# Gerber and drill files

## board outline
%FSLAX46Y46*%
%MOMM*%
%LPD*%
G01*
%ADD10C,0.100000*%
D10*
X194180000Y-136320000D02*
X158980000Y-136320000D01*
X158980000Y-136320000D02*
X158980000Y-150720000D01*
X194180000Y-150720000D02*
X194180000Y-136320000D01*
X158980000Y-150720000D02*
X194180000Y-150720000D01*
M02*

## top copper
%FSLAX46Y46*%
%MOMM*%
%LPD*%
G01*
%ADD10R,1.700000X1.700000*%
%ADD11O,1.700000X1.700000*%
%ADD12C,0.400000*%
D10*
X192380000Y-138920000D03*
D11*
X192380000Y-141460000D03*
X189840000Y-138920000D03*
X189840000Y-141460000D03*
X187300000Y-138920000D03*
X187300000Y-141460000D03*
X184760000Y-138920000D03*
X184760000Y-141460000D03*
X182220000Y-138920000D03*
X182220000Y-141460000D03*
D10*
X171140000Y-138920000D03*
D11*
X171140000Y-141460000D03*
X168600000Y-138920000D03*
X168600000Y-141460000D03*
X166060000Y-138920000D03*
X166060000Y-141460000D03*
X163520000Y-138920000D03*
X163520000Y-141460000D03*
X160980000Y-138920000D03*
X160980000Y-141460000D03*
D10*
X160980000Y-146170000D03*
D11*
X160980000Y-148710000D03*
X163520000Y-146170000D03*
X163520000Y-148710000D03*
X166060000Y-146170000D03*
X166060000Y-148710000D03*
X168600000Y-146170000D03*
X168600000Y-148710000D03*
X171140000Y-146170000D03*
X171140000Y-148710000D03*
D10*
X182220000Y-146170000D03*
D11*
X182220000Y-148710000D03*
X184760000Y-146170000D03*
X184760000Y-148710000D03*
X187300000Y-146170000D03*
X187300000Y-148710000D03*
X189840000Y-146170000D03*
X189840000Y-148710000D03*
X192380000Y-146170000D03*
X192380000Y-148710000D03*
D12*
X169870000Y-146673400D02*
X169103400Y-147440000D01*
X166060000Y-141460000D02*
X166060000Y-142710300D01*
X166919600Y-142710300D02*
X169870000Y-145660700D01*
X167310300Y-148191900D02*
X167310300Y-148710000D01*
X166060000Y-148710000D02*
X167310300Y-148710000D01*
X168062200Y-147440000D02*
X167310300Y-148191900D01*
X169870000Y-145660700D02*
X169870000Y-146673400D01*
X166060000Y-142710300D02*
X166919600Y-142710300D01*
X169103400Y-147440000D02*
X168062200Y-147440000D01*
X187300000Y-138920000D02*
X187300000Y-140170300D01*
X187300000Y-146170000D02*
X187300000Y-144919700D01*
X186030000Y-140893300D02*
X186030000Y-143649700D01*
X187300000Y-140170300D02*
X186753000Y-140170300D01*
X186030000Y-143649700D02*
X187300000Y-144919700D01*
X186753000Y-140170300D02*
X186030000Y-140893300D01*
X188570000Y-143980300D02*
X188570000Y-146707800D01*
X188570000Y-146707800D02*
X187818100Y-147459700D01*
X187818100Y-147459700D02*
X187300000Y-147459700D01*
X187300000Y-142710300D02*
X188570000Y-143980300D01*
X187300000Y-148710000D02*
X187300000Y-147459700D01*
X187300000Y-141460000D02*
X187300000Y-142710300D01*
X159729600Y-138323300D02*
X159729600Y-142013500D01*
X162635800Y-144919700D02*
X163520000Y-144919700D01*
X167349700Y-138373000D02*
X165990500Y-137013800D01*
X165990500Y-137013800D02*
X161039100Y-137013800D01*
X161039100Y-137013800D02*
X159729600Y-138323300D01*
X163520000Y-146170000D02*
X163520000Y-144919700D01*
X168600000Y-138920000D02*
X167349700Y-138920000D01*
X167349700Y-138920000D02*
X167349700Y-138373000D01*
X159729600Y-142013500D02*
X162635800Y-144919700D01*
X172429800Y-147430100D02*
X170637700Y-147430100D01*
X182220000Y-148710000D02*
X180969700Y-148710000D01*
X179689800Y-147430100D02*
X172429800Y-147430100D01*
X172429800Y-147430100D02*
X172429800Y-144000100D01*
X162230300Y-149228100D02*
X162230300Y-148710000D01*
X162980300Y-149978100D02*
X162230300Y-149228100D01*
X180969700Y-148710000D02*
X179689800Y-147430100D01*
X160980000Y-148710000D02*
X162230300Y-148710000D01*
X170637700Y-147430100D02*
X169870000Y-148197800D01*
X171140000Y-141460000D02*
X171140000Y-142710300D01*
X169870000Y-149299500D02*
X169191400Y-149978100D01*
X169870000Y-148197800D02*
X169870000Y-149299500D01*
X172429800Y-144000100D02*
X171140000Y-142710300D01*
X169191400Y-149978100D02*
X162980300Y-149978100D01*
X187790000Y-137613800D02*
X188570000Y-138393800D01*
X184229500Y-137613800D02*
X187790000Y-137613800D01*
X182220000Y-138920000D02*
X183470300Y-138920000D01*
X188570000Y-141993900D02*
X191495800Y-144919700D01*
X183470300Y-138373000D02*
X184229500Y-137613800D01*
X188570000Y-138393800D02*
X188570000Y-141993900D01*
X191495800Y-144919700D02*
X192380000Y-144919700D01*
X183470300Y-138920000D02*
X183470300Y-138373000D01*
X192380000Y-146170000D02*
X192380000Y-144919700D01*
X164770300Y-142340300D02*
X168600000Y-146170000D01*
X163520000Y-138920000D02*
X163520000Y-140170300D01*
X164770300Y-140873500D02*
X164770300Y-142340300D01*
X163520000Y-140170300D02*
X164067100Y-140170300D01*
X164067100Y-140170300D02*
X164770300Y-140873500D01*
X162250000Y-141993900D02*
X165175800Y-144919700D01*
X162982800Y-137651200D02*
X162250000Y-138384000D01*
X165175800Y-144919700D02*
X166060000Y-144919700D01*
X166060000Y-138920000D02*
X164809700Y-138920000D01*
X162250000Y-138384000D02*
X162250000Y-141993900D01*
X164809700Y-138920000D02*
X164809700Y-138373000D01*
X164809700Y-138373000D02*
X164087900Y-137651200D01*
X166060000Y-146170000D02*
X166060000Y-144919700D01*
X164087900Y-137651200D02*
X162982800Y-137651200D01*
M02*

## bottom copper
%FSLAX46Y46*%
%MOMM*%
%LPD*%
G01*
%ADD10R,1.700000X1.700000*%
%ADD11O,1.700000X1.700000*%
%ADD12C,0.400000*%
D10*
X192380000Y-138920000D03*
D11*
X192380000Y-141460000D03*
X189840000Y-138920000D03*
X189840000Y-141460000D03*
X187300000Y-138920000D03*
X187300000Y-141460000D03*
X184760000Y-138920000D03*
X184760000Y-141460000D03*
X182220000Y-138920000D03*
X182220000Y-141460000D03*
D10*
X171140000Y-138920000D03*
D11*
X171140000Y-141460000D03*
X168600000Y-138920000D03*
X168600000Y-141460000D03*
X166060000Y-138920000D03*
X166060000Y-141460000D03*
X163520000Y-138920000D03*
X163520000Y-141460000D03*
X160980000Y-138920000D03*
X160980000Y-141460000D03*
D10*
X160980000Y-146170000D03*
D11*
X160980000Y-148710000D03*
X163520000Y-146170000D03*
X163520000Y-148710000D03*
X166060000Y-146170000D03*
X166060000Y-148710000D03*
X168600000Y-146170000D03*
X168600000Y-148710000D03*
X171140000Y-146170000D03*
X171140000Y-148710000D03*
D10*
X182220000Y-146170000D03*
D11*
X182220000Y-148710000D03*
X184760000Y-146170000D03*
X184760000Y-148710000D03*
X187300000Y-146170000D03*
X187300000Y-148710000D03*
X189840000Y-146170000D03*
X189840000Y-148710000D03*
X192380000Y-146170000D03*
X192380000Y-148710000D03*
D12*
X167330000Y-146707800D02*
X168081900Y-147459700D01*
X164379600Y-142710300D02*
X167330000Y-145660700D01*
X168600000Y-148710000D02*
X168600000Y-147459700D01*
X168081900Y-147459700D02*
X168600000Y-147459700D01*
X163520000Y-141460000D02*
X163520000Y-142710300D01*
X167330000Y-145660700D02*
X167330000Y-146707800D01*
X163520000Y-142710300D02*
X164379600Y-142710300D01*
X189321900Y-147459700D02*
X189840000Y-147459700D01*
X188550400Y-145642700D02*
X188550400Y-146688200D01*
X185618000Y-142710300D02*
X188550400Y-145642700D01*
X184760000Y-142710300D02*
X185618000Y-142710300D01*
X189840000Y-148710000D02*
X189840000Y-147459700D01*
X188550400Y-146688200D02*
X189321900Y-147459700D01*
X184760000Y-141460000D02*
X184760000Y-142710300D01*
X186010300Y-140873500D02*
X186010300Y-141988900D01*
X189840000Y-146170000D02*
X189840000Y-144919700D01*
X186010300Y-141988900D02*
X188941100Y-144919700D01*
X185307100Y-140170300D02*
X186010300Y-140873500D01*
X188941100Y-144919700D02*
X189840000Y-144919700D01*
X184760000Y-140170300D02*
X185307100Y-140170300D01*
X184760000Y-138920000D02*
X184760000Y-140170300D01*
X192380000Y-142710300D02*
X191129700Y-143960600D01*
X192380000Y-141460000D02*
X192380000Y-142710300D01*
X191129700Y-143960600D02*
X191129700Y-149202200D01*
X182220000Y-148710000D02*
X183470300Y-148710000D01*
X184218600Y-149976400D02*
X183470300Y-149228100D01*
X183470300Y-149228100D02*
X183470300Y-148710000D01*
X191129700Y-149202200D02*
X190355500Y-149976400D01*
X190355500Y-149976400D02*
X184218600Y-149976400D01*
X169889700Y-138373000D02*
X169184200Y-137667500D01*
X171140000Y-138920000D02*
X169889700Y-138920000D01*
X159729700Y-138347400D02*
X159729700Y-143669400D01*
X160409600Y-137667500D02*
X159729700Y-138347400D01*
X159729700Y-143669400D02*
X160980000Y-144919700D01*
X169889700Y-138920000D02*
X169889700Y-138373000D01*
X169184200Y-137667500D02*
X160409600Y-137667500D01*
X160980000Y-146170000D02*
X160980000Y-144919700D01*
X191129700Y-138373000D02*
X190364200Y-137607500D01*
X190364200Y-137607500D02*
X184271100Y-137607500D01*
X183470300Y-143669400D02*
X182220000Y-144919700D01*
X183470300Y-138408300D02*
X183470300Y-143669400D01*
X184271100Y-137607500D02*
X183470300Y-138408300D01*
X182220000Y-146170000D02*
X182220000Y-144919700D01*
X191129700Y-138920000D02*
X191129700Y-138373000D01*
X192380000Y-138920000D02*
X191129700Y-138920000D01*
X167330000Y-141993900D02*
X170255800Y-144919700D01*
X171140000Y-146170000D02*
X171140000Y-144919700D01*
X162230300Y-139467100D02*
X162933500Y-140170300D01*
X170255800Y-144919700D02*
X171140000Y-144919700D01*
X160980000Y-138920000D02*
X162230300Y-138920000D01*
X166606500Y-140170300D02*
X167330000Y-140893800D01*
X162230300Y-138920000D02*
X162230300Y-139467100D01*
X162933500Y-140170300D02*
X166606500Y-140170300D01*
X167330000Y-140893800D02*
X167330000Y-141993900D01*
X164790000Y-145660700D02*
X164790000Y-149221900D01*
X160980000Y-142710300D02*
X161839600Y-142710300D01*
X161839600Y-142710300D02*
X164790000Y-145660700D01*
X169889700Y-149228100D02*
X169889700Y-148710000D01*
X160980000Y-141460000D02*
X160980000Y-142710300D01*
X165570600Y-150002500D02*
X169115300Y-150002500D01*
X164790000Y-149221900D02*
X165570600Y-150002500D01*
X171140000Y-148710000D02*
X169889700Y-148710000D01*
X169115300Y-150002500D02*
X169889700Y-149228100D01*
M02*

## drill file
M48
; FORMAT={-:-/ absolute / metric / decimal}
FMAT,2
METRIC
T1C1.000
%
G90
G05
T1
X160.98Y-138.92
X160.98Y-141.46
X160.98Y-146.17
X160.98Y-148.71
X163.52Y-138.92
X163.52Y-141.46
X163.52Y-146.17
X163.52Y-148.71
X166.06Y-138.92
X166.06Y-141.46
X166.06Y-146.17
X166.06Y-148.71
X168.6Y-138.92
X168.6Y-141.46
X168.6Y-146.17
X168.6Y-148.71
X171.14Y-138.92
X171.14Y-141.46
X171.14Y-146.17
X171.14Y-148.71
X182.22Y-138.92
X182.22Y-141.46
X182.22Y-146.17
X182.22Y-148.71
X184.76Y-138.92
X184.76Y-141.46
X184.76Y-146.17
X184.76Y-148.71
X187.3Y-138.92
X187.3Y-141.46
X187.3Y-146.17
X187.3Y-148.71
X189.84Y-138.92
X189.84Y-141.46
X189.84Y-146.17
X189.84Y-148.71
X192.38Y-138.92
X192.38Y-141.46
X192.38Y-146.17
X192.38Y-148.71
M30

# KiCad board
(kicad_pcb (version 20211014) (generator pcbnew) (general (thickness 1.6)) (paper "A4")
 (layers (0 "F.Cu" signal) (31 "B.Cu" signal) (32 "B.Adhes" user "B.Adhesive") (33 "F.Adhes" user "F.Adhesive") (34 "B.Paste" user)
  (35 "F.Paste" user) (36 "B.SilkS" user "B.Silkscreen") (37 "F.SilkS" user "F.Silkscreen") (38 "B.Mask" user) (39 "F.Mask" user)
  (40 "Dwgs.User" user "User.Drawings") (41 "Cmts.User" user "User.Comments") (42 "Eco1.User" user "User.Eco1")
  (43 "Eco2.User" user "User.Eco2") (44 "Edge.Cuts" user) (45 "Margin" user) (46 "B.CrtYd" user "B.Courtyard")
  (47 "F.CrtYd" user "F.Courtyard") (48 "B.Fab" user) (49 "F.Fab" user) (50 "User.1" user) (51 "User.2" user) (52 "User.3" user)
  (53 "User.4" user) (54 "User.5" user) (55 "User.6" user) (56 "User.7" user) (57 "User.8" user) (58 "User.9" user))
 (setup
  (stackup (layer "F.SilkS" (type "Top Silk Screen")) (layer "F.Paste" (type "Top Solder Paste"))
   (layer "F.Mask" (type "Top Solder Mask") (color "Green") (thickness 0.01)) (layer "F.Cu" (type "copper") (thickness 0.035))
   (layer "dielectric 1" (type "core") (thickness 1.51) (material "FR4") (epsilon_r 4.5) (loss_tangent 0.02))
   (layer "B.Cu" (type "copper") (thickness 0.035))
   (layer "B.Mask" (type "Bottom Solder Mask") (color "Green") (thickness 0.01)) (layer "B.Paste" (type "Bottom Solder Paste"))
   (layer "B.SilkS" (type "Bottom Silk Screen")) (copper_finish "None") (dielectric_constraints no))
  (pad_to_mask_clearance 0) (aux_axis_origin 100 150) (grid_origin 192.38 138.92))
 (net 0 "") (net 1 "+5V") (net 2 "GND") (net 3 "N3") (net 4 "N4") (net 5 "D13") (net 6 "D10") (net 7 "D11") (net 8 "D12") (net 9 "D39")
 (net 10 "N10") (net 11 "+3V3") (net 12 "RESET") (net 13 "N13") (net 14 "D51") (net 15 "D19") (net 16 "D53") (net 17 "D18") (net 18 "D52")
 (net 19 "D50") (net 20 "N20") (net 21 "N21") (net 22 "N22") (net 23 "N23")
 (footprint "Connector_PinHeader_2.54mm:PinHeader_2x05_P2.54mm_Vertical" (layer "F.Cu") (at 192.38 138.92 -90)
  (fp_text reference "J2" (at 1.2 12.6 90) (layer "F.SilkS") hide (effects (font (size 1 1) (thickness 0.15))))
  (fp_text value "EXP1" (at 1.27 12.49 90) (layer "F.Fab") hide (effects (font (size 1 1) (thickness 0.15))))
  (pad "1" thru_hole rect locked (at 0 0 270) (size 1.7 1.7) (drill 1) (layers *.Cu *.Mask) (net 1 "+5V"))
  (pad "2" thru_hole oval locked (at 2.54 0 270) (size 1.7 1.7) (drill 1) (layers *.Cu *.Mask) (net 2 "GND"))
  (pad "3" thru_hole oval locked (at 0 2.54 270) (size 1.7 1.7) (drill 1) (layers *.Cu *.Mask) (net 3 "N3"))
  (pad "4" thru_hole oval locked (at 2.54 2.54 270) (size 1.7 1.7) (drill 1) (layers *.Cu *.Mask) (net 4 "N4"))
  (pad "5" thru_hole oval locked (at 0 5.08 270) (size 1.7 1.7) (drill 1) (layers *.Cu *.Mask) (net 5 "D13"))
  (pad "6" thru_hole oval locked (at 2.54 5.08 270) (size 1.7 1.7) (drill 1) (layers *.Cu *.Mask) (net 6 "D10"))
  (pad "7" thru_hole oval locked (at 0 7.62 270) (size 1.7 1.7) (drill 1) (layers *.Cu *.Mask) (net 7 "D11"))
  (pad "8" thru_hole oval locked (at 2.54 7.62 270) (size 1.7 1.7) (drill 1) (layers *.Cu *.Mask) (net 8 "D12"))
  (pad "9" thru_hole oval locked (at 0 10.16 270) (size 1.7 1.7) (drill 1) (layers *.Cu *.Mask) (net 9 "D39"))
  (pad "10" thru_hole oval locked (at 2.54 10.16 270) (size 1.7 1.7) (drill 1) (layers *.Cu *.Mask) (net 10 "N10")))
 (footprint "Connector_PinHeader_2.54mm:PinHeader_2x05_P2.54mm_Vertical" (layer "F.Cu") (at 171.14 138.92 -90)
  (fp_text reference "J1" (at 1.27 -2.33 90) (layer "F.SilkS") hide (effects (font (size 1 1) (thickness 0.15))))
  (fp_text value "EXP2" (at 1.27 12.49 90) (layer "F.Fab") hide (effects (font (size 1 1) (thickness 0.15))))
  (pad "1" thru_hole rect locked (at 0 0 270) (size 1.7 1.7) (drill 1) (layers *.Cu *.Mask) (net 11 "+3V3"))
  (pad "2" thru_hole oval locked (at 2.54 0 270) (size 1.7 1.7) (drill 1) (layers *.Cu *.Mask) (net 2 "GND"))
  (pad "3" thru_hole oval locked (at 0 2.54 270) (size 1.7 1.7) (drill 1) (layers *.Cu *.Mask) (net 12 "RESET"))
  (pad "4" thru_hole oval locked (at 2.54 2.54 270) (size 1.7 1.7) (drill 1) (layers *.Cu *.Mask) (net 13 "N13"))
  (pad "5" thru_hole oval locked (at 0 5.08 270) (size 1.7 1.7) (drill 1) (layers *.Cu *.Mask) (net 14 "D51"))
  (pad "6" thru_hole oval locked (at 2.54 5.08 270) (size 1.7 1.7) (drill 1) (layers *.Cu *.Mask) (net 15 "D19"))
  (pad "7" thru_hole oval locked (at 0 7.62 270) (size 1.7 1.7) (drill 1) (layers *.Cu *.Mask) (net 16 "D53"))
  (pad "8" thru_hole oval locked (at 2.54 7.62 270) (size 1.7 1.7) (drill 1) (layers *.Cu *.Mask) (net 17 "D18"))
  (pad "9" thru_hole oval locked (at 0 10.16 270) (size 1.7 1.7) (drill 1) (layers *.Cu *.Mask) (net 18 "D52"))
  (pad "10" thru_hole oval locked (at 2.54 10.16 270) (size 1.7 1.7) (drill 1) (layers *.Cu *.Mask) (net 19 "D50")))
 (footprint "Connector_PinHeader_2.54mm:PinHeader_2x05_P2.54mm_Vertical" (layer "B.Cu") (at 160.98 146.17 -90)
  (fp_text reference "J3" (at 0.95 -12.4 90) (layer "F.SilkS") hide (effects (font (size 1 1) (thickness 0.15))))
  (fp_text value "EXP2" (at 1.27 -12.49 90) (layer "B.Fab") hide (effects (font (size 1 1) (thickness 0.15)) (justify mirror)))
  (pad "1" thru_hole rect locked (at 0 0 270) (size 1.7 1.7) (drill 1) (layers *.Cu *.Mask) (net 11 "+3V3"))
  (pad "2" thru_hole oval locked (at 2.54 0 270) (size 1.7 1.7) (drill 1) (layers *.Cu *.Mask) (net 2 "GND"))
  (pad "3" thru_hole oval locked (at 0 -2.54 270) (size 1.7 1.7) (drill 1) (layers *.Cu *.Mask) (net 12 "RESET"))
  (pad "4" thru_hole oval locked (at 2.54 -2.54 270) (size 1.7 1.7) (drill 1) (layers *.Cu *.Mask) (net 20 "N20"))
  (pad "5" thru_hole oval locked (at 0 -5.08 270) (size 1.7 1.7) (drill 1) (layers *.Cu *.Mask) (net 14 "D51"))
  (pad "6" thru_hole oval locked (at 2.54 -5.08 270) (size 1.7 1.7) (drill 1) (layers *.Cu *.Mask) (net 15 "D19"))
  (pad "7" thru_hole oval locked (at 0 -7.62 270) (size 1.7 1.7) (drill 1) (layers *.Cu *.Mask) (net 16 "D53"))
  (pad "8" thru_hole oval locked (at 2.54 -7.62 270) (size 1.7 1.7) (drill 1) (layers *.Cu *.Mask) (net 17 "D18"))
  (pad "9" thru_hole oval locked (at 0 -10.16 270) (size 1.7 1.7) (drill 1) (layers *.Cu *.Mask) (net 18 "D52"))
  (pad "10" thru_hole oval locked (at 2.54 -10.16 270) (size 1.7 1.7) (drill 1) (layers *.Cu *.Mask) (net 19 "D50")))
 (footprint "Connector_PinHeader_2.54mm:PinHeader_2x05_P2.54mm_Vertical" (layer "B.Cu") (at 182.22 146.17 -90)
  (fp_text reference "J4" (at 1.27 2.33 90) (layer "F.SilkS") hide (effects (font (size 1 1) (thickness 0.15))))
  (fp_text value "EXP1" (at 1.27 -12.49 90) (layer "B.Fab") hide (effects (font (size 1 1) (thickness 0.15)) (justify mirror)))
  (pad "1" thru_hole rect locked (at 0 0 270) (size 1.7 1.7) (drill 1) (layers *.Cu *.Mask) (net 1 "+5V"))
  (pad "2" thru_hole oval locked (at 2.54 0 270) (size 1.7 1.7) (drill 1) (layers *.Cu *.Mask) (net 2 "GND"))
  (pad "3" thru_hole oval locked (at 0 -2.54 270) (size 1.7 1.7) (drill 1) (layers *.Cu *.Mask) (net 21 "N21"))
  (pad "4" thru_hole oval locked (at 2.54 -2.54 270) (size 1.7 1.7) (drill 1) (layers *.Cu *.Mask) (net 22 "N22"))
  (pad "5" thru_hole oval locked (at 0 -5.08 270) (size 1.7 1.7) (drill 1) (layers *.Cu *.Mask) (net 5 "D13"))
  (pad "6" thru_hole oval locked (at 2.54 -5.08 270) (size 1.7 1.7) (drill 1) (layers *.Cu *.Mask) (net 6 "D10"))
  (pad "7" thru_hole oval locked (at 0 -7.62 270) (size 1.7 1.7) (drill 1) (layers *.Cu *.Mask) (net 7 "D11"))
  (pad "8" thru_hole oval locked (at 2.54 -7.62 270) (size 1.7 1.7) (drill 1) (layers *.Cu *.Mask) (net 8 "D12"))
  (pad "9" thru_hole oval locked (at 0 -10.16 270) (size 1.7 1.7) (drill 1) (layers *.Cu *.Mask) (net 9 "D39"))
  (pad "10" thru_hole oval locked (at 2.54 -10.16 270) (size 1.7 1.7) (drill 1) (layers *.Cu *.Mask) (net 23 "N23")))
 (gr_line (start 194.18 136.32) (end 158.98 136.32) (layer "Edge.Cuts") (width 0.1))
 (gr_line (start 158.98 136.32) (end 158.98 150.72) (layer "Edge.Cuts") (width 0.1))
 (gr_line (start 194.18 150.72) (end 194.18 136.32) (layer "Edge.Cuts") (width 0.1))
 (gr_line (start 158.98 150.72) (end 194.18 150.72) (layer "Edge.Cuts") (width 0.1))
 (segment (start 167.33 146.7078) (end 168.0819 147.4597) (width 0.4) (layer "B.Cu") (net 17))
 (segment (start 164.3796 142.7103) (end 167.33 145.6607) (width 0.4) (layer "B.Cu") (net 17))
 (segment (start 168.6 148.71) (end 168.6 147.4597) (width 0.4) (layer "B.Cu") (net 17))
 (segment (start 168.0819 147.4597) (end 168.6 147.4597) (width 0.4) (layer "B.Cu") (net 17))
 (segment (start 163.52 141.46) (end 163.52 142.7103) (width 0.4) (layer "B.Cu") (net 17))
 (segment (start 167.33 145.6607) (end 167.33 146.7078) (width 0.4) (layer "B.Cu") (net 17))
 (segment (start 163.52 142.7103) (end 164.3796 142.7103) (width 0.4) (layer "B.Cu") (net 17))
 (segment (start 169.87 146.6734) (end 169.1034 147.44) (width 0.4) (layer "F.Cu") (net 15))
 (segment (start 166.06 141.46) (end 166.06 142.7103) (width 0.4) (layer "F.Cu") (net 15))
 (segment (start 166.9196 142.7103) (end 169.87 145.6607) (width 0.4) (layer "F.Cu") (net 15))
 (segment (start 167.3103 148.1919) (end 167.3103 148.71) (width 0.4) (layer "F.Cu") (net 15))
 (segment (start 166.06 148.71) (end 167.3103 148.71) (width 0.4) (layer "F.Cu") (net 15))
 (segment (start 168.0622 147.44) (end 167.3103 148.1919) (width 0.4) (layer "F.Cu") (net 15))
 (segment (start 169.87 145.6607) (end 169.87 146.6734) (width 0.4) (layer "F.Cu") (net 15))
 (segment (start 166.06 142.7103) (end 166.9196 142.7103) (width 0.4) (layer "F.Cu") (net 15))
 (segment (start 169.1034 147.44) (end 168.0622 147.44) (width 0.4) (layer "F.Cu") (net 15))
 (segment (start 189.3219 147.4597) (end 189.84 147.4597) (width 0.4) (layer "B.Cu") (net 8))
 (segment (start 188.5504 145.6427) (end 188.5504 146.6882) (width 0.4) (layer "B.Cu") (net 8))
 (segment (start 185.618 142.7103) (end 188.5504 145.6427) (width 0.4) (layer "B.Cu") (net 8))
 (segment (start 184.76 142.7103) (end 185.618 142.7103) (width 0.4) (layer "B.Cu") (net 8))
 (segment (start 189.84 148.71) (end 189.84 147.4597) (width 0.4) (layer "B.Cu") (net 8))
 (segment (start 188.5504 146.6882) (end 189.3219 147.4597) (width 0.4) (layer "B.Cu") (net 8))
 (segment (start 184.76 141.46) (end 184.76 142.7103) (width 0.4) (layer "B.Cu") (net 8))
 (segment (start 187.3 138.92) (end 187.3 140.1703) (width 0.4) (layer "F.Cu") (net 5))
 (segment (start 187.3 146.17) (end 187.3 144.9197) (width 0.4) (layer "F.Cu") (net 5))
 (segment (start 186.03 140.8933) (end 186.03 143.6497) (width 0.4) (layer "F.Cu") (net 5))
 (segment (start 187.3 140.1703) (end 186.753 140.1703) (width 0.4) (layer "F.Cu") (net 5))
 (segment (start 186.03 143.6497) (end 187.3 144.9197) (width 0.4) (layer "F.Cu") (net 5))
 (segment (start 186.753 140.1703) (end 186.03 140.8933) (width 0.4) (layer "F.Cu") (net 5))
 (segment (start 188.57 143.9803) (end 188.57 146.7078) (width 0.4) (layer "F.Cu") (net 6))
 (segment (start 188.57 146.7078) (end 187.8181 147.4597) (width 0.4) (layer "F.Cu") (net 6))
 (segment (start 187.8181 147.4597) (end 187.3 147.4597) (width 0.4) (layer "F.Cu") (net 6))
 (segment (start 187.3 142.7103) (end 188.57 143.9803) (width 0.4) (layer "F.Cu") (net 6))
 (segment (start 187.3 148.71) (end 187.3 147.4597) (width 0.4) (layer "F.Cu") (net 6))
 (segment (start 187.3 141.46) (end 187.3 142.7103) (width 0.4) (layer "F.Cu") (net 6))
 (segment (start 186.0103 140.8735) (end 186.0103 141.9889) (width 0.4) (layer "B.Cu") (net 7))
 (segment (start 189.84 146.17) (end 189.84 144.9197) (width 0.4) (layer "B.Cu") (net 7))
 (segment (start 186.0103 141.9889) (end 188.9411 144.9197) (width 0.4) (layer "B.Cu") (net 7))
 (segment (start 185.3071 140.1703) (end 186.0103 140.8735) (width 0.4) (layer "B.Cu") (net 7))
 (segment (start 188.9411 144.9197) (end 189.84 144.9197) (width 0.4) (layer "B.Cu") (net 7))
 (segment (start 184.76 140.1703) (end 185.3071 140.1703) (width 0.4) (layer "B.Cu") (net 7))
 (segment (start 184.76 138.92) (end 184.76 140.1703) (width 0.4) (layer "B.Cu") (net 7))
 (segment (start 159.7296 138.3233) (end 159.7296 142.0135) (width 0.4) (layer "F.Cu") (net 12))
 (segment (start 162.6358 144.9197) (end 163.52 144.9197) (width 0.4) (layer "F.Cu") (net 12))
 (segment (start 167.3497 138.373) (end 165.9905 137.0138) (width 0.4) (layer "F.Cu") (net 12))
 (segment (start 165.9905 137.0138) (end 161.0391 137.0138) (width 0.4) (layer "F.Cu") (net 12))
 (segment (start 161.0391 137.0138) (end 159.7296 138.3233) (width 0.4) (layer "F.Cu") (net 12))
 (segment (start 163.52 146.17) (end 163.52 144.9197) (width 0.4) (layer "F.Cu") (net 12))
 (segment (start 168.6 138.92) (end 167.3497 138.92) (width 0.4) (layer "F.Cu") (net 12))
 (segment (start 167.3497 138.92) (end 167.3497 138.373) (width 0.4) (layer "F.Cu") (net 12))
 (segment (start 159.7296 142.0135) (end 162.6358 144.9197) (width 0.4) (layer "F.Cu") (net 12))
 (segment (start 172.4298 147.4301) (end 170.6377 147.4301) (width 0.4) (layer "F.Cu") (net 2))
 (segment (start 182.22 148.71) (end 180.9697 148.71) (width 0.4) (layer "F.Cu") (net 2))
 (segment (start 179.6898 147.4301) (end 172.4298 147.4301) (width 0.4) (layer "F.Cu") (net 2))
 (segment (start 172.4298 147.4301) (end 172.4298 144.0001) (width 0.4) (layer "F.Cu") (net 2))
 (segment (start 162.2303 149.2281) (end 162.2303 148.71) (width 0.4) (layer "F.Cu") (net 2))
 (segment (start 162.9803 149.9781) (end 162.2303 149.2281) (width 0.4) (layer "F.Cu") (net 2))
 (segment (start 180.9697 148.71) (end 179.6898 147.4301) (width 0.4) (layer "F.Cu") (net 2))
 (segment (start 160.98 148.71) (end 162.2303 148.71) (width 0.4) (layer "F.Cu") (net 2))
 (segment (start 170.6377 147.4301) (end 169.87 148.1978) (width 0.4) (layer "F.Cu") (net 2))
 (segment (start 171.14 141.46) (end 171.14 142.7103) (width 0.4) (layer "F.Cu") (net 2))
 (segment (start 169.87 149.2995) (end 169.1914 149.9781) (width 0.4) (layer "F.Cu") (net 2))
 (segment (start 169.87 148.1978) (end 169.87 149.2995) (width 0.4) (layer "F.Cu") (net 2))
 (segment (start 172.4298 144.0001) (end 171.14 142.7103) (width 0.4) (layer "F.Cu") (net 2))
 (segment (start 169.1914 149.9781) (end 162.9803 149.9781) (width 0.4) (layer "F.Cu") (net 2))
 (segment (start 192.38 142.7103) (end 191.1297 143.9606) (width 0.4) (layer "B.Cu") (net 2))
 (segment (start 192.38 141.46) (end 192.38 142.7103) (width 0.4) (layer "B.Cu") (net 2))
 (segment (start 191.1297 143.9606) (end 191.1297 149.2022) (width 0.4) (layer "B.Cu") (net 2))
 (segment (start 182.22 148.71) (end 183.4703 148.71) (width 0.4) (layer "B.Cu") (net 2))
 (segment (start 184.2186 149.9764) (end 183.4703 149.2281) (width 0.4) (layer "B.Cu") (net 2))
 (segment (start 183.4703 149.2281) (end 183.4703 148.71) (width 0.4) (layer "B.Cu") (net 2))
 (segment (start 191.1297 149.2022) (end 190.3555 149.9764) (width 0.4) (layer "B.Cu") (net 2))
 (segment (start 190.3555 149.9764) (end 184.2186 149.9764) (width 0.4) (layer "B.Cu") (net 2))
 (segment (start 187.79 137.6138) (end 188.57 138.3938) (width 0.4) (layer "F.Cu") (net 9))
 (segment (start 184.2295 137.6138) (end 187.79 137.6138) (width 0.4) (layer "F.Cu") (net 9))
 (segment (start 182.22 138.92) (end 183.4703 138.92) (width 0.4) (layer "F.Cu") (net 9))
 (segment (start 188.57 141.9939) (end 191.4958 144.9197) (width 0.4) (layer "F.Cu") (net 9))
 (segment (start 183.4703 138.373) (end 184.2295 137.6138) (width 0.4) (layer "F.Cu") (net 9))
 (segment (start 188.57 138.3938) (end 188.57 141.9939) (width 0.4) (layer "F.Cu") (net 9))
 (segment (start 191.4958 144.9197) (end 192.38 144.9197) (width 0.4) (layer "F.Cu") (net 9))
 (segment (start 183.4703 138.92) (end 183.4703 138.373) (width 0.4) (layer "F.Cu") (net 9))
 (segment (start 192.38 146.17) (end 192.38 144.9197) (width 0.4) (layer "F.Cu") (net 9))
 (segment (start 169.8897 138.373) (end 169.1842 137.6675) (width 0.4) (layer "B.Cu") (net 11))
 (segment (start 171.14 138.92) (end 169.8897 138.92) (width 0.4) (layer "B.Cu") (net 11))
 (segment (start 159.7297 138.3474) (end 159.7297 143.6694) (width 0.4) (layer "B.Cu") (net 11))
 (segment (start 160.4096 137.6675) (end 159.7297 138.3474) (width 0.4) (layer "B.Cu") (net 11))
 (segment (start 159.7297 143.6694) (end 160.98 144.9197) (width 0.4) (layer "B.Cu") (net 11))
 (segment (start 169.8897 138.92) (end 169.8897 138.373) (width 0.4) (layer "B.Cu") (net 11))
 (segment (start 169.1842 137.6675) (end 160.4096 137.6675) (width 0.4) (layer "B.Cu") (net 11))
 (segment (start 160.98 146.17) (end 160.98 144.9197) (width 0.4) (layer "B.Cu") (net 11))
 (segment (start 191.1297 138.373) (end 190.3642 137.6075) (width 0.4) (layer "B.Cu") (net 1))
 (segment (start 190.3642 137.6075) (end 184.2711 137.6075) (width 0.4) (layer "B.Cu") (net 1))
 (segment (start 183.4703 143.6694) (end 182.22 144.9197) (width 0.4) (layer "B.Cu") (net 1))
 (segment (start 183.4703 138.4083) (end 183.4703 143.6694) (width 0.4) (layer "B.Cu") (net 1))
 (segment (start 184.2711 137.6075) (end 183.4703 138.4083) (width 0.4) (layer "B.Cu") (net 1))
 (segment (start 182.22 146.17) (end 182.22 144.9197) (width 0.4) (layer "B.Cu") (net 1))
 (segment (start 191.1297 138.92) (end 191.1297 138.373) (width 0.4) (layer "B.Cu") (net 1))
 (segment (start 192.38 138.92) (end 191.1297 138.92) (width 0.4) (layer "B.Cu") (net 1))
 (segment (start 164.7703 142.3403) (end 168.6 146.17) (width 0.4) (layer "F.Cu") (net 16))
 (segment (start 163.52 138.92) (end 163.52 140.1703) (width 0.4) (layer "F.Cu") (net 16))
 (segment (start 164.7703 140.8735) (end 164.7703 142.3403) (width 0.4) (layer "F.Cu") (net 16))
 (segment (start 163.52 140.1703) (end 164.0671 140.1703) (width 0.4) (layer "F.Cu") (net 16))
 (segment (start 164.0671 140.1703) (end 164.7703 140.8735) (width 0.4) (layer "F.Cu") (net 16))
 (segment (start 167.33 141.9939) (end 170.2558 144.9197) (width 0.4) (layer "B.Cu") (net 18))
 (segment (start 171.14 146.17) (end 171.14 144.9197) (width 0.4) (layer "B.Cu") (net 18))
 (segment (start 162.2303 139.4671) (end 162.9335 140.1703) (width 0.4) (layer "B.Cu") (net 18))
 (segment (start 170.2558 144.9197) (end 171.14 144.9197) (width 0.4) (layer "B.Cu") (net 18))
 (segment (start 160.98 138.92) (end 162.2303 138.92) (width 0.4) (layer "B.Cu") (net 18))
 (segment (start 166.6065 140.1703) (end 167.33 140.8938) (width 0.4) (layer "B.Cu") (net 18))
 (segment (start 162.2303 138.92) (end 162.2303 139.4671) (width 0.4) (layer "B.Cu") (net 18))
 (segment (start 162.9335 140.1703) (end 166.6065 140.1703) (width 0.4) (layer "B.Cu") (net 18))
 (segment (start 167.33 140.8938) (end 167.33 141.9939) (width 0.4) (layer "B.Cu") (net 18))
 (segment (start 162.25 141.9939) (end 165.1758 144.9197) (width 0.4) (layer "F.Cu") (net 14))
 (segment (start 162.9828 137.6512) (end 162.25 138.384) (width 0.4) (layer "F.Cu") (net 14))
 (segment (start 165.1758 144.9197) (end 166.06 144.9197) (width 0.4) (layer "F.Cu") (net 14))
 (segment (start 166.06 138.92) (end 164.8097 138.92) (width 0.4) (layer "F.Cu") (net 14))
 (segment (start 162.25 138.384) (end 162.25 141.9939) (width 0.4) (layer "F.Cu") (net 14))
 (segment (start 164.8097 138.92) (end 164.8097 138.373) (width 0.4) (layer "F.Cu") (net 14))
 (segment (start 164.8097 138.373) (end 164.0879 137.6512) (width 0.4) (layer "F.Cu") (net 14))
 (segment (start 166.06 146.17) (end 166.06 144.9197) (width 0.4) (layer "F.Cu") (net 14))
 (segment (start 164.0879 137.6512) (end 162.9828 137.6512) (width 0.4) (layer "F.Cu") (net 14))
 (segment (start 164.79 145.6607) (end 164.79 149.2219) (width 0.4) (layer "B.Cu") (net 19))
 (segment (start 160.98 142.7103) (end 161.8396 142.7103) (width 0.4) (layer "B.Cu") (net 19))
 (segment (start 161.8396 142.7103) (end 164.79 145.6607) (width 0.4) (layer "B.Cu") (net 19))
 (segment (start 169.8897 149.2281) (end 169.8897 148.71) (width 0.4) (layer "B.Cu") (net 19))
 (segment (start 160.98 141.46) (end 160.98 142.7103) (width 0.4) (layer "B.Cu") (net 19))
 (segment (start 165.5706 150.0025) (end 169.1153 150.0025) (width 0.4) (layer "B.Cu") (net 19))
 (segment (start 164.79 149.2219) (end 165.5706 150.0025) (width 0.4) (layer "B.Cu") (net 19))
 (segment (start 171.14 148.71) (end 169.8897 148.71) (width 0.4) (layer "B.Cu") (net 19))
 (segment (start 169.1153 150.0025) (end 169.8897 149.2281) (width 0.4) (layer "B.Cu") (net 19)))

